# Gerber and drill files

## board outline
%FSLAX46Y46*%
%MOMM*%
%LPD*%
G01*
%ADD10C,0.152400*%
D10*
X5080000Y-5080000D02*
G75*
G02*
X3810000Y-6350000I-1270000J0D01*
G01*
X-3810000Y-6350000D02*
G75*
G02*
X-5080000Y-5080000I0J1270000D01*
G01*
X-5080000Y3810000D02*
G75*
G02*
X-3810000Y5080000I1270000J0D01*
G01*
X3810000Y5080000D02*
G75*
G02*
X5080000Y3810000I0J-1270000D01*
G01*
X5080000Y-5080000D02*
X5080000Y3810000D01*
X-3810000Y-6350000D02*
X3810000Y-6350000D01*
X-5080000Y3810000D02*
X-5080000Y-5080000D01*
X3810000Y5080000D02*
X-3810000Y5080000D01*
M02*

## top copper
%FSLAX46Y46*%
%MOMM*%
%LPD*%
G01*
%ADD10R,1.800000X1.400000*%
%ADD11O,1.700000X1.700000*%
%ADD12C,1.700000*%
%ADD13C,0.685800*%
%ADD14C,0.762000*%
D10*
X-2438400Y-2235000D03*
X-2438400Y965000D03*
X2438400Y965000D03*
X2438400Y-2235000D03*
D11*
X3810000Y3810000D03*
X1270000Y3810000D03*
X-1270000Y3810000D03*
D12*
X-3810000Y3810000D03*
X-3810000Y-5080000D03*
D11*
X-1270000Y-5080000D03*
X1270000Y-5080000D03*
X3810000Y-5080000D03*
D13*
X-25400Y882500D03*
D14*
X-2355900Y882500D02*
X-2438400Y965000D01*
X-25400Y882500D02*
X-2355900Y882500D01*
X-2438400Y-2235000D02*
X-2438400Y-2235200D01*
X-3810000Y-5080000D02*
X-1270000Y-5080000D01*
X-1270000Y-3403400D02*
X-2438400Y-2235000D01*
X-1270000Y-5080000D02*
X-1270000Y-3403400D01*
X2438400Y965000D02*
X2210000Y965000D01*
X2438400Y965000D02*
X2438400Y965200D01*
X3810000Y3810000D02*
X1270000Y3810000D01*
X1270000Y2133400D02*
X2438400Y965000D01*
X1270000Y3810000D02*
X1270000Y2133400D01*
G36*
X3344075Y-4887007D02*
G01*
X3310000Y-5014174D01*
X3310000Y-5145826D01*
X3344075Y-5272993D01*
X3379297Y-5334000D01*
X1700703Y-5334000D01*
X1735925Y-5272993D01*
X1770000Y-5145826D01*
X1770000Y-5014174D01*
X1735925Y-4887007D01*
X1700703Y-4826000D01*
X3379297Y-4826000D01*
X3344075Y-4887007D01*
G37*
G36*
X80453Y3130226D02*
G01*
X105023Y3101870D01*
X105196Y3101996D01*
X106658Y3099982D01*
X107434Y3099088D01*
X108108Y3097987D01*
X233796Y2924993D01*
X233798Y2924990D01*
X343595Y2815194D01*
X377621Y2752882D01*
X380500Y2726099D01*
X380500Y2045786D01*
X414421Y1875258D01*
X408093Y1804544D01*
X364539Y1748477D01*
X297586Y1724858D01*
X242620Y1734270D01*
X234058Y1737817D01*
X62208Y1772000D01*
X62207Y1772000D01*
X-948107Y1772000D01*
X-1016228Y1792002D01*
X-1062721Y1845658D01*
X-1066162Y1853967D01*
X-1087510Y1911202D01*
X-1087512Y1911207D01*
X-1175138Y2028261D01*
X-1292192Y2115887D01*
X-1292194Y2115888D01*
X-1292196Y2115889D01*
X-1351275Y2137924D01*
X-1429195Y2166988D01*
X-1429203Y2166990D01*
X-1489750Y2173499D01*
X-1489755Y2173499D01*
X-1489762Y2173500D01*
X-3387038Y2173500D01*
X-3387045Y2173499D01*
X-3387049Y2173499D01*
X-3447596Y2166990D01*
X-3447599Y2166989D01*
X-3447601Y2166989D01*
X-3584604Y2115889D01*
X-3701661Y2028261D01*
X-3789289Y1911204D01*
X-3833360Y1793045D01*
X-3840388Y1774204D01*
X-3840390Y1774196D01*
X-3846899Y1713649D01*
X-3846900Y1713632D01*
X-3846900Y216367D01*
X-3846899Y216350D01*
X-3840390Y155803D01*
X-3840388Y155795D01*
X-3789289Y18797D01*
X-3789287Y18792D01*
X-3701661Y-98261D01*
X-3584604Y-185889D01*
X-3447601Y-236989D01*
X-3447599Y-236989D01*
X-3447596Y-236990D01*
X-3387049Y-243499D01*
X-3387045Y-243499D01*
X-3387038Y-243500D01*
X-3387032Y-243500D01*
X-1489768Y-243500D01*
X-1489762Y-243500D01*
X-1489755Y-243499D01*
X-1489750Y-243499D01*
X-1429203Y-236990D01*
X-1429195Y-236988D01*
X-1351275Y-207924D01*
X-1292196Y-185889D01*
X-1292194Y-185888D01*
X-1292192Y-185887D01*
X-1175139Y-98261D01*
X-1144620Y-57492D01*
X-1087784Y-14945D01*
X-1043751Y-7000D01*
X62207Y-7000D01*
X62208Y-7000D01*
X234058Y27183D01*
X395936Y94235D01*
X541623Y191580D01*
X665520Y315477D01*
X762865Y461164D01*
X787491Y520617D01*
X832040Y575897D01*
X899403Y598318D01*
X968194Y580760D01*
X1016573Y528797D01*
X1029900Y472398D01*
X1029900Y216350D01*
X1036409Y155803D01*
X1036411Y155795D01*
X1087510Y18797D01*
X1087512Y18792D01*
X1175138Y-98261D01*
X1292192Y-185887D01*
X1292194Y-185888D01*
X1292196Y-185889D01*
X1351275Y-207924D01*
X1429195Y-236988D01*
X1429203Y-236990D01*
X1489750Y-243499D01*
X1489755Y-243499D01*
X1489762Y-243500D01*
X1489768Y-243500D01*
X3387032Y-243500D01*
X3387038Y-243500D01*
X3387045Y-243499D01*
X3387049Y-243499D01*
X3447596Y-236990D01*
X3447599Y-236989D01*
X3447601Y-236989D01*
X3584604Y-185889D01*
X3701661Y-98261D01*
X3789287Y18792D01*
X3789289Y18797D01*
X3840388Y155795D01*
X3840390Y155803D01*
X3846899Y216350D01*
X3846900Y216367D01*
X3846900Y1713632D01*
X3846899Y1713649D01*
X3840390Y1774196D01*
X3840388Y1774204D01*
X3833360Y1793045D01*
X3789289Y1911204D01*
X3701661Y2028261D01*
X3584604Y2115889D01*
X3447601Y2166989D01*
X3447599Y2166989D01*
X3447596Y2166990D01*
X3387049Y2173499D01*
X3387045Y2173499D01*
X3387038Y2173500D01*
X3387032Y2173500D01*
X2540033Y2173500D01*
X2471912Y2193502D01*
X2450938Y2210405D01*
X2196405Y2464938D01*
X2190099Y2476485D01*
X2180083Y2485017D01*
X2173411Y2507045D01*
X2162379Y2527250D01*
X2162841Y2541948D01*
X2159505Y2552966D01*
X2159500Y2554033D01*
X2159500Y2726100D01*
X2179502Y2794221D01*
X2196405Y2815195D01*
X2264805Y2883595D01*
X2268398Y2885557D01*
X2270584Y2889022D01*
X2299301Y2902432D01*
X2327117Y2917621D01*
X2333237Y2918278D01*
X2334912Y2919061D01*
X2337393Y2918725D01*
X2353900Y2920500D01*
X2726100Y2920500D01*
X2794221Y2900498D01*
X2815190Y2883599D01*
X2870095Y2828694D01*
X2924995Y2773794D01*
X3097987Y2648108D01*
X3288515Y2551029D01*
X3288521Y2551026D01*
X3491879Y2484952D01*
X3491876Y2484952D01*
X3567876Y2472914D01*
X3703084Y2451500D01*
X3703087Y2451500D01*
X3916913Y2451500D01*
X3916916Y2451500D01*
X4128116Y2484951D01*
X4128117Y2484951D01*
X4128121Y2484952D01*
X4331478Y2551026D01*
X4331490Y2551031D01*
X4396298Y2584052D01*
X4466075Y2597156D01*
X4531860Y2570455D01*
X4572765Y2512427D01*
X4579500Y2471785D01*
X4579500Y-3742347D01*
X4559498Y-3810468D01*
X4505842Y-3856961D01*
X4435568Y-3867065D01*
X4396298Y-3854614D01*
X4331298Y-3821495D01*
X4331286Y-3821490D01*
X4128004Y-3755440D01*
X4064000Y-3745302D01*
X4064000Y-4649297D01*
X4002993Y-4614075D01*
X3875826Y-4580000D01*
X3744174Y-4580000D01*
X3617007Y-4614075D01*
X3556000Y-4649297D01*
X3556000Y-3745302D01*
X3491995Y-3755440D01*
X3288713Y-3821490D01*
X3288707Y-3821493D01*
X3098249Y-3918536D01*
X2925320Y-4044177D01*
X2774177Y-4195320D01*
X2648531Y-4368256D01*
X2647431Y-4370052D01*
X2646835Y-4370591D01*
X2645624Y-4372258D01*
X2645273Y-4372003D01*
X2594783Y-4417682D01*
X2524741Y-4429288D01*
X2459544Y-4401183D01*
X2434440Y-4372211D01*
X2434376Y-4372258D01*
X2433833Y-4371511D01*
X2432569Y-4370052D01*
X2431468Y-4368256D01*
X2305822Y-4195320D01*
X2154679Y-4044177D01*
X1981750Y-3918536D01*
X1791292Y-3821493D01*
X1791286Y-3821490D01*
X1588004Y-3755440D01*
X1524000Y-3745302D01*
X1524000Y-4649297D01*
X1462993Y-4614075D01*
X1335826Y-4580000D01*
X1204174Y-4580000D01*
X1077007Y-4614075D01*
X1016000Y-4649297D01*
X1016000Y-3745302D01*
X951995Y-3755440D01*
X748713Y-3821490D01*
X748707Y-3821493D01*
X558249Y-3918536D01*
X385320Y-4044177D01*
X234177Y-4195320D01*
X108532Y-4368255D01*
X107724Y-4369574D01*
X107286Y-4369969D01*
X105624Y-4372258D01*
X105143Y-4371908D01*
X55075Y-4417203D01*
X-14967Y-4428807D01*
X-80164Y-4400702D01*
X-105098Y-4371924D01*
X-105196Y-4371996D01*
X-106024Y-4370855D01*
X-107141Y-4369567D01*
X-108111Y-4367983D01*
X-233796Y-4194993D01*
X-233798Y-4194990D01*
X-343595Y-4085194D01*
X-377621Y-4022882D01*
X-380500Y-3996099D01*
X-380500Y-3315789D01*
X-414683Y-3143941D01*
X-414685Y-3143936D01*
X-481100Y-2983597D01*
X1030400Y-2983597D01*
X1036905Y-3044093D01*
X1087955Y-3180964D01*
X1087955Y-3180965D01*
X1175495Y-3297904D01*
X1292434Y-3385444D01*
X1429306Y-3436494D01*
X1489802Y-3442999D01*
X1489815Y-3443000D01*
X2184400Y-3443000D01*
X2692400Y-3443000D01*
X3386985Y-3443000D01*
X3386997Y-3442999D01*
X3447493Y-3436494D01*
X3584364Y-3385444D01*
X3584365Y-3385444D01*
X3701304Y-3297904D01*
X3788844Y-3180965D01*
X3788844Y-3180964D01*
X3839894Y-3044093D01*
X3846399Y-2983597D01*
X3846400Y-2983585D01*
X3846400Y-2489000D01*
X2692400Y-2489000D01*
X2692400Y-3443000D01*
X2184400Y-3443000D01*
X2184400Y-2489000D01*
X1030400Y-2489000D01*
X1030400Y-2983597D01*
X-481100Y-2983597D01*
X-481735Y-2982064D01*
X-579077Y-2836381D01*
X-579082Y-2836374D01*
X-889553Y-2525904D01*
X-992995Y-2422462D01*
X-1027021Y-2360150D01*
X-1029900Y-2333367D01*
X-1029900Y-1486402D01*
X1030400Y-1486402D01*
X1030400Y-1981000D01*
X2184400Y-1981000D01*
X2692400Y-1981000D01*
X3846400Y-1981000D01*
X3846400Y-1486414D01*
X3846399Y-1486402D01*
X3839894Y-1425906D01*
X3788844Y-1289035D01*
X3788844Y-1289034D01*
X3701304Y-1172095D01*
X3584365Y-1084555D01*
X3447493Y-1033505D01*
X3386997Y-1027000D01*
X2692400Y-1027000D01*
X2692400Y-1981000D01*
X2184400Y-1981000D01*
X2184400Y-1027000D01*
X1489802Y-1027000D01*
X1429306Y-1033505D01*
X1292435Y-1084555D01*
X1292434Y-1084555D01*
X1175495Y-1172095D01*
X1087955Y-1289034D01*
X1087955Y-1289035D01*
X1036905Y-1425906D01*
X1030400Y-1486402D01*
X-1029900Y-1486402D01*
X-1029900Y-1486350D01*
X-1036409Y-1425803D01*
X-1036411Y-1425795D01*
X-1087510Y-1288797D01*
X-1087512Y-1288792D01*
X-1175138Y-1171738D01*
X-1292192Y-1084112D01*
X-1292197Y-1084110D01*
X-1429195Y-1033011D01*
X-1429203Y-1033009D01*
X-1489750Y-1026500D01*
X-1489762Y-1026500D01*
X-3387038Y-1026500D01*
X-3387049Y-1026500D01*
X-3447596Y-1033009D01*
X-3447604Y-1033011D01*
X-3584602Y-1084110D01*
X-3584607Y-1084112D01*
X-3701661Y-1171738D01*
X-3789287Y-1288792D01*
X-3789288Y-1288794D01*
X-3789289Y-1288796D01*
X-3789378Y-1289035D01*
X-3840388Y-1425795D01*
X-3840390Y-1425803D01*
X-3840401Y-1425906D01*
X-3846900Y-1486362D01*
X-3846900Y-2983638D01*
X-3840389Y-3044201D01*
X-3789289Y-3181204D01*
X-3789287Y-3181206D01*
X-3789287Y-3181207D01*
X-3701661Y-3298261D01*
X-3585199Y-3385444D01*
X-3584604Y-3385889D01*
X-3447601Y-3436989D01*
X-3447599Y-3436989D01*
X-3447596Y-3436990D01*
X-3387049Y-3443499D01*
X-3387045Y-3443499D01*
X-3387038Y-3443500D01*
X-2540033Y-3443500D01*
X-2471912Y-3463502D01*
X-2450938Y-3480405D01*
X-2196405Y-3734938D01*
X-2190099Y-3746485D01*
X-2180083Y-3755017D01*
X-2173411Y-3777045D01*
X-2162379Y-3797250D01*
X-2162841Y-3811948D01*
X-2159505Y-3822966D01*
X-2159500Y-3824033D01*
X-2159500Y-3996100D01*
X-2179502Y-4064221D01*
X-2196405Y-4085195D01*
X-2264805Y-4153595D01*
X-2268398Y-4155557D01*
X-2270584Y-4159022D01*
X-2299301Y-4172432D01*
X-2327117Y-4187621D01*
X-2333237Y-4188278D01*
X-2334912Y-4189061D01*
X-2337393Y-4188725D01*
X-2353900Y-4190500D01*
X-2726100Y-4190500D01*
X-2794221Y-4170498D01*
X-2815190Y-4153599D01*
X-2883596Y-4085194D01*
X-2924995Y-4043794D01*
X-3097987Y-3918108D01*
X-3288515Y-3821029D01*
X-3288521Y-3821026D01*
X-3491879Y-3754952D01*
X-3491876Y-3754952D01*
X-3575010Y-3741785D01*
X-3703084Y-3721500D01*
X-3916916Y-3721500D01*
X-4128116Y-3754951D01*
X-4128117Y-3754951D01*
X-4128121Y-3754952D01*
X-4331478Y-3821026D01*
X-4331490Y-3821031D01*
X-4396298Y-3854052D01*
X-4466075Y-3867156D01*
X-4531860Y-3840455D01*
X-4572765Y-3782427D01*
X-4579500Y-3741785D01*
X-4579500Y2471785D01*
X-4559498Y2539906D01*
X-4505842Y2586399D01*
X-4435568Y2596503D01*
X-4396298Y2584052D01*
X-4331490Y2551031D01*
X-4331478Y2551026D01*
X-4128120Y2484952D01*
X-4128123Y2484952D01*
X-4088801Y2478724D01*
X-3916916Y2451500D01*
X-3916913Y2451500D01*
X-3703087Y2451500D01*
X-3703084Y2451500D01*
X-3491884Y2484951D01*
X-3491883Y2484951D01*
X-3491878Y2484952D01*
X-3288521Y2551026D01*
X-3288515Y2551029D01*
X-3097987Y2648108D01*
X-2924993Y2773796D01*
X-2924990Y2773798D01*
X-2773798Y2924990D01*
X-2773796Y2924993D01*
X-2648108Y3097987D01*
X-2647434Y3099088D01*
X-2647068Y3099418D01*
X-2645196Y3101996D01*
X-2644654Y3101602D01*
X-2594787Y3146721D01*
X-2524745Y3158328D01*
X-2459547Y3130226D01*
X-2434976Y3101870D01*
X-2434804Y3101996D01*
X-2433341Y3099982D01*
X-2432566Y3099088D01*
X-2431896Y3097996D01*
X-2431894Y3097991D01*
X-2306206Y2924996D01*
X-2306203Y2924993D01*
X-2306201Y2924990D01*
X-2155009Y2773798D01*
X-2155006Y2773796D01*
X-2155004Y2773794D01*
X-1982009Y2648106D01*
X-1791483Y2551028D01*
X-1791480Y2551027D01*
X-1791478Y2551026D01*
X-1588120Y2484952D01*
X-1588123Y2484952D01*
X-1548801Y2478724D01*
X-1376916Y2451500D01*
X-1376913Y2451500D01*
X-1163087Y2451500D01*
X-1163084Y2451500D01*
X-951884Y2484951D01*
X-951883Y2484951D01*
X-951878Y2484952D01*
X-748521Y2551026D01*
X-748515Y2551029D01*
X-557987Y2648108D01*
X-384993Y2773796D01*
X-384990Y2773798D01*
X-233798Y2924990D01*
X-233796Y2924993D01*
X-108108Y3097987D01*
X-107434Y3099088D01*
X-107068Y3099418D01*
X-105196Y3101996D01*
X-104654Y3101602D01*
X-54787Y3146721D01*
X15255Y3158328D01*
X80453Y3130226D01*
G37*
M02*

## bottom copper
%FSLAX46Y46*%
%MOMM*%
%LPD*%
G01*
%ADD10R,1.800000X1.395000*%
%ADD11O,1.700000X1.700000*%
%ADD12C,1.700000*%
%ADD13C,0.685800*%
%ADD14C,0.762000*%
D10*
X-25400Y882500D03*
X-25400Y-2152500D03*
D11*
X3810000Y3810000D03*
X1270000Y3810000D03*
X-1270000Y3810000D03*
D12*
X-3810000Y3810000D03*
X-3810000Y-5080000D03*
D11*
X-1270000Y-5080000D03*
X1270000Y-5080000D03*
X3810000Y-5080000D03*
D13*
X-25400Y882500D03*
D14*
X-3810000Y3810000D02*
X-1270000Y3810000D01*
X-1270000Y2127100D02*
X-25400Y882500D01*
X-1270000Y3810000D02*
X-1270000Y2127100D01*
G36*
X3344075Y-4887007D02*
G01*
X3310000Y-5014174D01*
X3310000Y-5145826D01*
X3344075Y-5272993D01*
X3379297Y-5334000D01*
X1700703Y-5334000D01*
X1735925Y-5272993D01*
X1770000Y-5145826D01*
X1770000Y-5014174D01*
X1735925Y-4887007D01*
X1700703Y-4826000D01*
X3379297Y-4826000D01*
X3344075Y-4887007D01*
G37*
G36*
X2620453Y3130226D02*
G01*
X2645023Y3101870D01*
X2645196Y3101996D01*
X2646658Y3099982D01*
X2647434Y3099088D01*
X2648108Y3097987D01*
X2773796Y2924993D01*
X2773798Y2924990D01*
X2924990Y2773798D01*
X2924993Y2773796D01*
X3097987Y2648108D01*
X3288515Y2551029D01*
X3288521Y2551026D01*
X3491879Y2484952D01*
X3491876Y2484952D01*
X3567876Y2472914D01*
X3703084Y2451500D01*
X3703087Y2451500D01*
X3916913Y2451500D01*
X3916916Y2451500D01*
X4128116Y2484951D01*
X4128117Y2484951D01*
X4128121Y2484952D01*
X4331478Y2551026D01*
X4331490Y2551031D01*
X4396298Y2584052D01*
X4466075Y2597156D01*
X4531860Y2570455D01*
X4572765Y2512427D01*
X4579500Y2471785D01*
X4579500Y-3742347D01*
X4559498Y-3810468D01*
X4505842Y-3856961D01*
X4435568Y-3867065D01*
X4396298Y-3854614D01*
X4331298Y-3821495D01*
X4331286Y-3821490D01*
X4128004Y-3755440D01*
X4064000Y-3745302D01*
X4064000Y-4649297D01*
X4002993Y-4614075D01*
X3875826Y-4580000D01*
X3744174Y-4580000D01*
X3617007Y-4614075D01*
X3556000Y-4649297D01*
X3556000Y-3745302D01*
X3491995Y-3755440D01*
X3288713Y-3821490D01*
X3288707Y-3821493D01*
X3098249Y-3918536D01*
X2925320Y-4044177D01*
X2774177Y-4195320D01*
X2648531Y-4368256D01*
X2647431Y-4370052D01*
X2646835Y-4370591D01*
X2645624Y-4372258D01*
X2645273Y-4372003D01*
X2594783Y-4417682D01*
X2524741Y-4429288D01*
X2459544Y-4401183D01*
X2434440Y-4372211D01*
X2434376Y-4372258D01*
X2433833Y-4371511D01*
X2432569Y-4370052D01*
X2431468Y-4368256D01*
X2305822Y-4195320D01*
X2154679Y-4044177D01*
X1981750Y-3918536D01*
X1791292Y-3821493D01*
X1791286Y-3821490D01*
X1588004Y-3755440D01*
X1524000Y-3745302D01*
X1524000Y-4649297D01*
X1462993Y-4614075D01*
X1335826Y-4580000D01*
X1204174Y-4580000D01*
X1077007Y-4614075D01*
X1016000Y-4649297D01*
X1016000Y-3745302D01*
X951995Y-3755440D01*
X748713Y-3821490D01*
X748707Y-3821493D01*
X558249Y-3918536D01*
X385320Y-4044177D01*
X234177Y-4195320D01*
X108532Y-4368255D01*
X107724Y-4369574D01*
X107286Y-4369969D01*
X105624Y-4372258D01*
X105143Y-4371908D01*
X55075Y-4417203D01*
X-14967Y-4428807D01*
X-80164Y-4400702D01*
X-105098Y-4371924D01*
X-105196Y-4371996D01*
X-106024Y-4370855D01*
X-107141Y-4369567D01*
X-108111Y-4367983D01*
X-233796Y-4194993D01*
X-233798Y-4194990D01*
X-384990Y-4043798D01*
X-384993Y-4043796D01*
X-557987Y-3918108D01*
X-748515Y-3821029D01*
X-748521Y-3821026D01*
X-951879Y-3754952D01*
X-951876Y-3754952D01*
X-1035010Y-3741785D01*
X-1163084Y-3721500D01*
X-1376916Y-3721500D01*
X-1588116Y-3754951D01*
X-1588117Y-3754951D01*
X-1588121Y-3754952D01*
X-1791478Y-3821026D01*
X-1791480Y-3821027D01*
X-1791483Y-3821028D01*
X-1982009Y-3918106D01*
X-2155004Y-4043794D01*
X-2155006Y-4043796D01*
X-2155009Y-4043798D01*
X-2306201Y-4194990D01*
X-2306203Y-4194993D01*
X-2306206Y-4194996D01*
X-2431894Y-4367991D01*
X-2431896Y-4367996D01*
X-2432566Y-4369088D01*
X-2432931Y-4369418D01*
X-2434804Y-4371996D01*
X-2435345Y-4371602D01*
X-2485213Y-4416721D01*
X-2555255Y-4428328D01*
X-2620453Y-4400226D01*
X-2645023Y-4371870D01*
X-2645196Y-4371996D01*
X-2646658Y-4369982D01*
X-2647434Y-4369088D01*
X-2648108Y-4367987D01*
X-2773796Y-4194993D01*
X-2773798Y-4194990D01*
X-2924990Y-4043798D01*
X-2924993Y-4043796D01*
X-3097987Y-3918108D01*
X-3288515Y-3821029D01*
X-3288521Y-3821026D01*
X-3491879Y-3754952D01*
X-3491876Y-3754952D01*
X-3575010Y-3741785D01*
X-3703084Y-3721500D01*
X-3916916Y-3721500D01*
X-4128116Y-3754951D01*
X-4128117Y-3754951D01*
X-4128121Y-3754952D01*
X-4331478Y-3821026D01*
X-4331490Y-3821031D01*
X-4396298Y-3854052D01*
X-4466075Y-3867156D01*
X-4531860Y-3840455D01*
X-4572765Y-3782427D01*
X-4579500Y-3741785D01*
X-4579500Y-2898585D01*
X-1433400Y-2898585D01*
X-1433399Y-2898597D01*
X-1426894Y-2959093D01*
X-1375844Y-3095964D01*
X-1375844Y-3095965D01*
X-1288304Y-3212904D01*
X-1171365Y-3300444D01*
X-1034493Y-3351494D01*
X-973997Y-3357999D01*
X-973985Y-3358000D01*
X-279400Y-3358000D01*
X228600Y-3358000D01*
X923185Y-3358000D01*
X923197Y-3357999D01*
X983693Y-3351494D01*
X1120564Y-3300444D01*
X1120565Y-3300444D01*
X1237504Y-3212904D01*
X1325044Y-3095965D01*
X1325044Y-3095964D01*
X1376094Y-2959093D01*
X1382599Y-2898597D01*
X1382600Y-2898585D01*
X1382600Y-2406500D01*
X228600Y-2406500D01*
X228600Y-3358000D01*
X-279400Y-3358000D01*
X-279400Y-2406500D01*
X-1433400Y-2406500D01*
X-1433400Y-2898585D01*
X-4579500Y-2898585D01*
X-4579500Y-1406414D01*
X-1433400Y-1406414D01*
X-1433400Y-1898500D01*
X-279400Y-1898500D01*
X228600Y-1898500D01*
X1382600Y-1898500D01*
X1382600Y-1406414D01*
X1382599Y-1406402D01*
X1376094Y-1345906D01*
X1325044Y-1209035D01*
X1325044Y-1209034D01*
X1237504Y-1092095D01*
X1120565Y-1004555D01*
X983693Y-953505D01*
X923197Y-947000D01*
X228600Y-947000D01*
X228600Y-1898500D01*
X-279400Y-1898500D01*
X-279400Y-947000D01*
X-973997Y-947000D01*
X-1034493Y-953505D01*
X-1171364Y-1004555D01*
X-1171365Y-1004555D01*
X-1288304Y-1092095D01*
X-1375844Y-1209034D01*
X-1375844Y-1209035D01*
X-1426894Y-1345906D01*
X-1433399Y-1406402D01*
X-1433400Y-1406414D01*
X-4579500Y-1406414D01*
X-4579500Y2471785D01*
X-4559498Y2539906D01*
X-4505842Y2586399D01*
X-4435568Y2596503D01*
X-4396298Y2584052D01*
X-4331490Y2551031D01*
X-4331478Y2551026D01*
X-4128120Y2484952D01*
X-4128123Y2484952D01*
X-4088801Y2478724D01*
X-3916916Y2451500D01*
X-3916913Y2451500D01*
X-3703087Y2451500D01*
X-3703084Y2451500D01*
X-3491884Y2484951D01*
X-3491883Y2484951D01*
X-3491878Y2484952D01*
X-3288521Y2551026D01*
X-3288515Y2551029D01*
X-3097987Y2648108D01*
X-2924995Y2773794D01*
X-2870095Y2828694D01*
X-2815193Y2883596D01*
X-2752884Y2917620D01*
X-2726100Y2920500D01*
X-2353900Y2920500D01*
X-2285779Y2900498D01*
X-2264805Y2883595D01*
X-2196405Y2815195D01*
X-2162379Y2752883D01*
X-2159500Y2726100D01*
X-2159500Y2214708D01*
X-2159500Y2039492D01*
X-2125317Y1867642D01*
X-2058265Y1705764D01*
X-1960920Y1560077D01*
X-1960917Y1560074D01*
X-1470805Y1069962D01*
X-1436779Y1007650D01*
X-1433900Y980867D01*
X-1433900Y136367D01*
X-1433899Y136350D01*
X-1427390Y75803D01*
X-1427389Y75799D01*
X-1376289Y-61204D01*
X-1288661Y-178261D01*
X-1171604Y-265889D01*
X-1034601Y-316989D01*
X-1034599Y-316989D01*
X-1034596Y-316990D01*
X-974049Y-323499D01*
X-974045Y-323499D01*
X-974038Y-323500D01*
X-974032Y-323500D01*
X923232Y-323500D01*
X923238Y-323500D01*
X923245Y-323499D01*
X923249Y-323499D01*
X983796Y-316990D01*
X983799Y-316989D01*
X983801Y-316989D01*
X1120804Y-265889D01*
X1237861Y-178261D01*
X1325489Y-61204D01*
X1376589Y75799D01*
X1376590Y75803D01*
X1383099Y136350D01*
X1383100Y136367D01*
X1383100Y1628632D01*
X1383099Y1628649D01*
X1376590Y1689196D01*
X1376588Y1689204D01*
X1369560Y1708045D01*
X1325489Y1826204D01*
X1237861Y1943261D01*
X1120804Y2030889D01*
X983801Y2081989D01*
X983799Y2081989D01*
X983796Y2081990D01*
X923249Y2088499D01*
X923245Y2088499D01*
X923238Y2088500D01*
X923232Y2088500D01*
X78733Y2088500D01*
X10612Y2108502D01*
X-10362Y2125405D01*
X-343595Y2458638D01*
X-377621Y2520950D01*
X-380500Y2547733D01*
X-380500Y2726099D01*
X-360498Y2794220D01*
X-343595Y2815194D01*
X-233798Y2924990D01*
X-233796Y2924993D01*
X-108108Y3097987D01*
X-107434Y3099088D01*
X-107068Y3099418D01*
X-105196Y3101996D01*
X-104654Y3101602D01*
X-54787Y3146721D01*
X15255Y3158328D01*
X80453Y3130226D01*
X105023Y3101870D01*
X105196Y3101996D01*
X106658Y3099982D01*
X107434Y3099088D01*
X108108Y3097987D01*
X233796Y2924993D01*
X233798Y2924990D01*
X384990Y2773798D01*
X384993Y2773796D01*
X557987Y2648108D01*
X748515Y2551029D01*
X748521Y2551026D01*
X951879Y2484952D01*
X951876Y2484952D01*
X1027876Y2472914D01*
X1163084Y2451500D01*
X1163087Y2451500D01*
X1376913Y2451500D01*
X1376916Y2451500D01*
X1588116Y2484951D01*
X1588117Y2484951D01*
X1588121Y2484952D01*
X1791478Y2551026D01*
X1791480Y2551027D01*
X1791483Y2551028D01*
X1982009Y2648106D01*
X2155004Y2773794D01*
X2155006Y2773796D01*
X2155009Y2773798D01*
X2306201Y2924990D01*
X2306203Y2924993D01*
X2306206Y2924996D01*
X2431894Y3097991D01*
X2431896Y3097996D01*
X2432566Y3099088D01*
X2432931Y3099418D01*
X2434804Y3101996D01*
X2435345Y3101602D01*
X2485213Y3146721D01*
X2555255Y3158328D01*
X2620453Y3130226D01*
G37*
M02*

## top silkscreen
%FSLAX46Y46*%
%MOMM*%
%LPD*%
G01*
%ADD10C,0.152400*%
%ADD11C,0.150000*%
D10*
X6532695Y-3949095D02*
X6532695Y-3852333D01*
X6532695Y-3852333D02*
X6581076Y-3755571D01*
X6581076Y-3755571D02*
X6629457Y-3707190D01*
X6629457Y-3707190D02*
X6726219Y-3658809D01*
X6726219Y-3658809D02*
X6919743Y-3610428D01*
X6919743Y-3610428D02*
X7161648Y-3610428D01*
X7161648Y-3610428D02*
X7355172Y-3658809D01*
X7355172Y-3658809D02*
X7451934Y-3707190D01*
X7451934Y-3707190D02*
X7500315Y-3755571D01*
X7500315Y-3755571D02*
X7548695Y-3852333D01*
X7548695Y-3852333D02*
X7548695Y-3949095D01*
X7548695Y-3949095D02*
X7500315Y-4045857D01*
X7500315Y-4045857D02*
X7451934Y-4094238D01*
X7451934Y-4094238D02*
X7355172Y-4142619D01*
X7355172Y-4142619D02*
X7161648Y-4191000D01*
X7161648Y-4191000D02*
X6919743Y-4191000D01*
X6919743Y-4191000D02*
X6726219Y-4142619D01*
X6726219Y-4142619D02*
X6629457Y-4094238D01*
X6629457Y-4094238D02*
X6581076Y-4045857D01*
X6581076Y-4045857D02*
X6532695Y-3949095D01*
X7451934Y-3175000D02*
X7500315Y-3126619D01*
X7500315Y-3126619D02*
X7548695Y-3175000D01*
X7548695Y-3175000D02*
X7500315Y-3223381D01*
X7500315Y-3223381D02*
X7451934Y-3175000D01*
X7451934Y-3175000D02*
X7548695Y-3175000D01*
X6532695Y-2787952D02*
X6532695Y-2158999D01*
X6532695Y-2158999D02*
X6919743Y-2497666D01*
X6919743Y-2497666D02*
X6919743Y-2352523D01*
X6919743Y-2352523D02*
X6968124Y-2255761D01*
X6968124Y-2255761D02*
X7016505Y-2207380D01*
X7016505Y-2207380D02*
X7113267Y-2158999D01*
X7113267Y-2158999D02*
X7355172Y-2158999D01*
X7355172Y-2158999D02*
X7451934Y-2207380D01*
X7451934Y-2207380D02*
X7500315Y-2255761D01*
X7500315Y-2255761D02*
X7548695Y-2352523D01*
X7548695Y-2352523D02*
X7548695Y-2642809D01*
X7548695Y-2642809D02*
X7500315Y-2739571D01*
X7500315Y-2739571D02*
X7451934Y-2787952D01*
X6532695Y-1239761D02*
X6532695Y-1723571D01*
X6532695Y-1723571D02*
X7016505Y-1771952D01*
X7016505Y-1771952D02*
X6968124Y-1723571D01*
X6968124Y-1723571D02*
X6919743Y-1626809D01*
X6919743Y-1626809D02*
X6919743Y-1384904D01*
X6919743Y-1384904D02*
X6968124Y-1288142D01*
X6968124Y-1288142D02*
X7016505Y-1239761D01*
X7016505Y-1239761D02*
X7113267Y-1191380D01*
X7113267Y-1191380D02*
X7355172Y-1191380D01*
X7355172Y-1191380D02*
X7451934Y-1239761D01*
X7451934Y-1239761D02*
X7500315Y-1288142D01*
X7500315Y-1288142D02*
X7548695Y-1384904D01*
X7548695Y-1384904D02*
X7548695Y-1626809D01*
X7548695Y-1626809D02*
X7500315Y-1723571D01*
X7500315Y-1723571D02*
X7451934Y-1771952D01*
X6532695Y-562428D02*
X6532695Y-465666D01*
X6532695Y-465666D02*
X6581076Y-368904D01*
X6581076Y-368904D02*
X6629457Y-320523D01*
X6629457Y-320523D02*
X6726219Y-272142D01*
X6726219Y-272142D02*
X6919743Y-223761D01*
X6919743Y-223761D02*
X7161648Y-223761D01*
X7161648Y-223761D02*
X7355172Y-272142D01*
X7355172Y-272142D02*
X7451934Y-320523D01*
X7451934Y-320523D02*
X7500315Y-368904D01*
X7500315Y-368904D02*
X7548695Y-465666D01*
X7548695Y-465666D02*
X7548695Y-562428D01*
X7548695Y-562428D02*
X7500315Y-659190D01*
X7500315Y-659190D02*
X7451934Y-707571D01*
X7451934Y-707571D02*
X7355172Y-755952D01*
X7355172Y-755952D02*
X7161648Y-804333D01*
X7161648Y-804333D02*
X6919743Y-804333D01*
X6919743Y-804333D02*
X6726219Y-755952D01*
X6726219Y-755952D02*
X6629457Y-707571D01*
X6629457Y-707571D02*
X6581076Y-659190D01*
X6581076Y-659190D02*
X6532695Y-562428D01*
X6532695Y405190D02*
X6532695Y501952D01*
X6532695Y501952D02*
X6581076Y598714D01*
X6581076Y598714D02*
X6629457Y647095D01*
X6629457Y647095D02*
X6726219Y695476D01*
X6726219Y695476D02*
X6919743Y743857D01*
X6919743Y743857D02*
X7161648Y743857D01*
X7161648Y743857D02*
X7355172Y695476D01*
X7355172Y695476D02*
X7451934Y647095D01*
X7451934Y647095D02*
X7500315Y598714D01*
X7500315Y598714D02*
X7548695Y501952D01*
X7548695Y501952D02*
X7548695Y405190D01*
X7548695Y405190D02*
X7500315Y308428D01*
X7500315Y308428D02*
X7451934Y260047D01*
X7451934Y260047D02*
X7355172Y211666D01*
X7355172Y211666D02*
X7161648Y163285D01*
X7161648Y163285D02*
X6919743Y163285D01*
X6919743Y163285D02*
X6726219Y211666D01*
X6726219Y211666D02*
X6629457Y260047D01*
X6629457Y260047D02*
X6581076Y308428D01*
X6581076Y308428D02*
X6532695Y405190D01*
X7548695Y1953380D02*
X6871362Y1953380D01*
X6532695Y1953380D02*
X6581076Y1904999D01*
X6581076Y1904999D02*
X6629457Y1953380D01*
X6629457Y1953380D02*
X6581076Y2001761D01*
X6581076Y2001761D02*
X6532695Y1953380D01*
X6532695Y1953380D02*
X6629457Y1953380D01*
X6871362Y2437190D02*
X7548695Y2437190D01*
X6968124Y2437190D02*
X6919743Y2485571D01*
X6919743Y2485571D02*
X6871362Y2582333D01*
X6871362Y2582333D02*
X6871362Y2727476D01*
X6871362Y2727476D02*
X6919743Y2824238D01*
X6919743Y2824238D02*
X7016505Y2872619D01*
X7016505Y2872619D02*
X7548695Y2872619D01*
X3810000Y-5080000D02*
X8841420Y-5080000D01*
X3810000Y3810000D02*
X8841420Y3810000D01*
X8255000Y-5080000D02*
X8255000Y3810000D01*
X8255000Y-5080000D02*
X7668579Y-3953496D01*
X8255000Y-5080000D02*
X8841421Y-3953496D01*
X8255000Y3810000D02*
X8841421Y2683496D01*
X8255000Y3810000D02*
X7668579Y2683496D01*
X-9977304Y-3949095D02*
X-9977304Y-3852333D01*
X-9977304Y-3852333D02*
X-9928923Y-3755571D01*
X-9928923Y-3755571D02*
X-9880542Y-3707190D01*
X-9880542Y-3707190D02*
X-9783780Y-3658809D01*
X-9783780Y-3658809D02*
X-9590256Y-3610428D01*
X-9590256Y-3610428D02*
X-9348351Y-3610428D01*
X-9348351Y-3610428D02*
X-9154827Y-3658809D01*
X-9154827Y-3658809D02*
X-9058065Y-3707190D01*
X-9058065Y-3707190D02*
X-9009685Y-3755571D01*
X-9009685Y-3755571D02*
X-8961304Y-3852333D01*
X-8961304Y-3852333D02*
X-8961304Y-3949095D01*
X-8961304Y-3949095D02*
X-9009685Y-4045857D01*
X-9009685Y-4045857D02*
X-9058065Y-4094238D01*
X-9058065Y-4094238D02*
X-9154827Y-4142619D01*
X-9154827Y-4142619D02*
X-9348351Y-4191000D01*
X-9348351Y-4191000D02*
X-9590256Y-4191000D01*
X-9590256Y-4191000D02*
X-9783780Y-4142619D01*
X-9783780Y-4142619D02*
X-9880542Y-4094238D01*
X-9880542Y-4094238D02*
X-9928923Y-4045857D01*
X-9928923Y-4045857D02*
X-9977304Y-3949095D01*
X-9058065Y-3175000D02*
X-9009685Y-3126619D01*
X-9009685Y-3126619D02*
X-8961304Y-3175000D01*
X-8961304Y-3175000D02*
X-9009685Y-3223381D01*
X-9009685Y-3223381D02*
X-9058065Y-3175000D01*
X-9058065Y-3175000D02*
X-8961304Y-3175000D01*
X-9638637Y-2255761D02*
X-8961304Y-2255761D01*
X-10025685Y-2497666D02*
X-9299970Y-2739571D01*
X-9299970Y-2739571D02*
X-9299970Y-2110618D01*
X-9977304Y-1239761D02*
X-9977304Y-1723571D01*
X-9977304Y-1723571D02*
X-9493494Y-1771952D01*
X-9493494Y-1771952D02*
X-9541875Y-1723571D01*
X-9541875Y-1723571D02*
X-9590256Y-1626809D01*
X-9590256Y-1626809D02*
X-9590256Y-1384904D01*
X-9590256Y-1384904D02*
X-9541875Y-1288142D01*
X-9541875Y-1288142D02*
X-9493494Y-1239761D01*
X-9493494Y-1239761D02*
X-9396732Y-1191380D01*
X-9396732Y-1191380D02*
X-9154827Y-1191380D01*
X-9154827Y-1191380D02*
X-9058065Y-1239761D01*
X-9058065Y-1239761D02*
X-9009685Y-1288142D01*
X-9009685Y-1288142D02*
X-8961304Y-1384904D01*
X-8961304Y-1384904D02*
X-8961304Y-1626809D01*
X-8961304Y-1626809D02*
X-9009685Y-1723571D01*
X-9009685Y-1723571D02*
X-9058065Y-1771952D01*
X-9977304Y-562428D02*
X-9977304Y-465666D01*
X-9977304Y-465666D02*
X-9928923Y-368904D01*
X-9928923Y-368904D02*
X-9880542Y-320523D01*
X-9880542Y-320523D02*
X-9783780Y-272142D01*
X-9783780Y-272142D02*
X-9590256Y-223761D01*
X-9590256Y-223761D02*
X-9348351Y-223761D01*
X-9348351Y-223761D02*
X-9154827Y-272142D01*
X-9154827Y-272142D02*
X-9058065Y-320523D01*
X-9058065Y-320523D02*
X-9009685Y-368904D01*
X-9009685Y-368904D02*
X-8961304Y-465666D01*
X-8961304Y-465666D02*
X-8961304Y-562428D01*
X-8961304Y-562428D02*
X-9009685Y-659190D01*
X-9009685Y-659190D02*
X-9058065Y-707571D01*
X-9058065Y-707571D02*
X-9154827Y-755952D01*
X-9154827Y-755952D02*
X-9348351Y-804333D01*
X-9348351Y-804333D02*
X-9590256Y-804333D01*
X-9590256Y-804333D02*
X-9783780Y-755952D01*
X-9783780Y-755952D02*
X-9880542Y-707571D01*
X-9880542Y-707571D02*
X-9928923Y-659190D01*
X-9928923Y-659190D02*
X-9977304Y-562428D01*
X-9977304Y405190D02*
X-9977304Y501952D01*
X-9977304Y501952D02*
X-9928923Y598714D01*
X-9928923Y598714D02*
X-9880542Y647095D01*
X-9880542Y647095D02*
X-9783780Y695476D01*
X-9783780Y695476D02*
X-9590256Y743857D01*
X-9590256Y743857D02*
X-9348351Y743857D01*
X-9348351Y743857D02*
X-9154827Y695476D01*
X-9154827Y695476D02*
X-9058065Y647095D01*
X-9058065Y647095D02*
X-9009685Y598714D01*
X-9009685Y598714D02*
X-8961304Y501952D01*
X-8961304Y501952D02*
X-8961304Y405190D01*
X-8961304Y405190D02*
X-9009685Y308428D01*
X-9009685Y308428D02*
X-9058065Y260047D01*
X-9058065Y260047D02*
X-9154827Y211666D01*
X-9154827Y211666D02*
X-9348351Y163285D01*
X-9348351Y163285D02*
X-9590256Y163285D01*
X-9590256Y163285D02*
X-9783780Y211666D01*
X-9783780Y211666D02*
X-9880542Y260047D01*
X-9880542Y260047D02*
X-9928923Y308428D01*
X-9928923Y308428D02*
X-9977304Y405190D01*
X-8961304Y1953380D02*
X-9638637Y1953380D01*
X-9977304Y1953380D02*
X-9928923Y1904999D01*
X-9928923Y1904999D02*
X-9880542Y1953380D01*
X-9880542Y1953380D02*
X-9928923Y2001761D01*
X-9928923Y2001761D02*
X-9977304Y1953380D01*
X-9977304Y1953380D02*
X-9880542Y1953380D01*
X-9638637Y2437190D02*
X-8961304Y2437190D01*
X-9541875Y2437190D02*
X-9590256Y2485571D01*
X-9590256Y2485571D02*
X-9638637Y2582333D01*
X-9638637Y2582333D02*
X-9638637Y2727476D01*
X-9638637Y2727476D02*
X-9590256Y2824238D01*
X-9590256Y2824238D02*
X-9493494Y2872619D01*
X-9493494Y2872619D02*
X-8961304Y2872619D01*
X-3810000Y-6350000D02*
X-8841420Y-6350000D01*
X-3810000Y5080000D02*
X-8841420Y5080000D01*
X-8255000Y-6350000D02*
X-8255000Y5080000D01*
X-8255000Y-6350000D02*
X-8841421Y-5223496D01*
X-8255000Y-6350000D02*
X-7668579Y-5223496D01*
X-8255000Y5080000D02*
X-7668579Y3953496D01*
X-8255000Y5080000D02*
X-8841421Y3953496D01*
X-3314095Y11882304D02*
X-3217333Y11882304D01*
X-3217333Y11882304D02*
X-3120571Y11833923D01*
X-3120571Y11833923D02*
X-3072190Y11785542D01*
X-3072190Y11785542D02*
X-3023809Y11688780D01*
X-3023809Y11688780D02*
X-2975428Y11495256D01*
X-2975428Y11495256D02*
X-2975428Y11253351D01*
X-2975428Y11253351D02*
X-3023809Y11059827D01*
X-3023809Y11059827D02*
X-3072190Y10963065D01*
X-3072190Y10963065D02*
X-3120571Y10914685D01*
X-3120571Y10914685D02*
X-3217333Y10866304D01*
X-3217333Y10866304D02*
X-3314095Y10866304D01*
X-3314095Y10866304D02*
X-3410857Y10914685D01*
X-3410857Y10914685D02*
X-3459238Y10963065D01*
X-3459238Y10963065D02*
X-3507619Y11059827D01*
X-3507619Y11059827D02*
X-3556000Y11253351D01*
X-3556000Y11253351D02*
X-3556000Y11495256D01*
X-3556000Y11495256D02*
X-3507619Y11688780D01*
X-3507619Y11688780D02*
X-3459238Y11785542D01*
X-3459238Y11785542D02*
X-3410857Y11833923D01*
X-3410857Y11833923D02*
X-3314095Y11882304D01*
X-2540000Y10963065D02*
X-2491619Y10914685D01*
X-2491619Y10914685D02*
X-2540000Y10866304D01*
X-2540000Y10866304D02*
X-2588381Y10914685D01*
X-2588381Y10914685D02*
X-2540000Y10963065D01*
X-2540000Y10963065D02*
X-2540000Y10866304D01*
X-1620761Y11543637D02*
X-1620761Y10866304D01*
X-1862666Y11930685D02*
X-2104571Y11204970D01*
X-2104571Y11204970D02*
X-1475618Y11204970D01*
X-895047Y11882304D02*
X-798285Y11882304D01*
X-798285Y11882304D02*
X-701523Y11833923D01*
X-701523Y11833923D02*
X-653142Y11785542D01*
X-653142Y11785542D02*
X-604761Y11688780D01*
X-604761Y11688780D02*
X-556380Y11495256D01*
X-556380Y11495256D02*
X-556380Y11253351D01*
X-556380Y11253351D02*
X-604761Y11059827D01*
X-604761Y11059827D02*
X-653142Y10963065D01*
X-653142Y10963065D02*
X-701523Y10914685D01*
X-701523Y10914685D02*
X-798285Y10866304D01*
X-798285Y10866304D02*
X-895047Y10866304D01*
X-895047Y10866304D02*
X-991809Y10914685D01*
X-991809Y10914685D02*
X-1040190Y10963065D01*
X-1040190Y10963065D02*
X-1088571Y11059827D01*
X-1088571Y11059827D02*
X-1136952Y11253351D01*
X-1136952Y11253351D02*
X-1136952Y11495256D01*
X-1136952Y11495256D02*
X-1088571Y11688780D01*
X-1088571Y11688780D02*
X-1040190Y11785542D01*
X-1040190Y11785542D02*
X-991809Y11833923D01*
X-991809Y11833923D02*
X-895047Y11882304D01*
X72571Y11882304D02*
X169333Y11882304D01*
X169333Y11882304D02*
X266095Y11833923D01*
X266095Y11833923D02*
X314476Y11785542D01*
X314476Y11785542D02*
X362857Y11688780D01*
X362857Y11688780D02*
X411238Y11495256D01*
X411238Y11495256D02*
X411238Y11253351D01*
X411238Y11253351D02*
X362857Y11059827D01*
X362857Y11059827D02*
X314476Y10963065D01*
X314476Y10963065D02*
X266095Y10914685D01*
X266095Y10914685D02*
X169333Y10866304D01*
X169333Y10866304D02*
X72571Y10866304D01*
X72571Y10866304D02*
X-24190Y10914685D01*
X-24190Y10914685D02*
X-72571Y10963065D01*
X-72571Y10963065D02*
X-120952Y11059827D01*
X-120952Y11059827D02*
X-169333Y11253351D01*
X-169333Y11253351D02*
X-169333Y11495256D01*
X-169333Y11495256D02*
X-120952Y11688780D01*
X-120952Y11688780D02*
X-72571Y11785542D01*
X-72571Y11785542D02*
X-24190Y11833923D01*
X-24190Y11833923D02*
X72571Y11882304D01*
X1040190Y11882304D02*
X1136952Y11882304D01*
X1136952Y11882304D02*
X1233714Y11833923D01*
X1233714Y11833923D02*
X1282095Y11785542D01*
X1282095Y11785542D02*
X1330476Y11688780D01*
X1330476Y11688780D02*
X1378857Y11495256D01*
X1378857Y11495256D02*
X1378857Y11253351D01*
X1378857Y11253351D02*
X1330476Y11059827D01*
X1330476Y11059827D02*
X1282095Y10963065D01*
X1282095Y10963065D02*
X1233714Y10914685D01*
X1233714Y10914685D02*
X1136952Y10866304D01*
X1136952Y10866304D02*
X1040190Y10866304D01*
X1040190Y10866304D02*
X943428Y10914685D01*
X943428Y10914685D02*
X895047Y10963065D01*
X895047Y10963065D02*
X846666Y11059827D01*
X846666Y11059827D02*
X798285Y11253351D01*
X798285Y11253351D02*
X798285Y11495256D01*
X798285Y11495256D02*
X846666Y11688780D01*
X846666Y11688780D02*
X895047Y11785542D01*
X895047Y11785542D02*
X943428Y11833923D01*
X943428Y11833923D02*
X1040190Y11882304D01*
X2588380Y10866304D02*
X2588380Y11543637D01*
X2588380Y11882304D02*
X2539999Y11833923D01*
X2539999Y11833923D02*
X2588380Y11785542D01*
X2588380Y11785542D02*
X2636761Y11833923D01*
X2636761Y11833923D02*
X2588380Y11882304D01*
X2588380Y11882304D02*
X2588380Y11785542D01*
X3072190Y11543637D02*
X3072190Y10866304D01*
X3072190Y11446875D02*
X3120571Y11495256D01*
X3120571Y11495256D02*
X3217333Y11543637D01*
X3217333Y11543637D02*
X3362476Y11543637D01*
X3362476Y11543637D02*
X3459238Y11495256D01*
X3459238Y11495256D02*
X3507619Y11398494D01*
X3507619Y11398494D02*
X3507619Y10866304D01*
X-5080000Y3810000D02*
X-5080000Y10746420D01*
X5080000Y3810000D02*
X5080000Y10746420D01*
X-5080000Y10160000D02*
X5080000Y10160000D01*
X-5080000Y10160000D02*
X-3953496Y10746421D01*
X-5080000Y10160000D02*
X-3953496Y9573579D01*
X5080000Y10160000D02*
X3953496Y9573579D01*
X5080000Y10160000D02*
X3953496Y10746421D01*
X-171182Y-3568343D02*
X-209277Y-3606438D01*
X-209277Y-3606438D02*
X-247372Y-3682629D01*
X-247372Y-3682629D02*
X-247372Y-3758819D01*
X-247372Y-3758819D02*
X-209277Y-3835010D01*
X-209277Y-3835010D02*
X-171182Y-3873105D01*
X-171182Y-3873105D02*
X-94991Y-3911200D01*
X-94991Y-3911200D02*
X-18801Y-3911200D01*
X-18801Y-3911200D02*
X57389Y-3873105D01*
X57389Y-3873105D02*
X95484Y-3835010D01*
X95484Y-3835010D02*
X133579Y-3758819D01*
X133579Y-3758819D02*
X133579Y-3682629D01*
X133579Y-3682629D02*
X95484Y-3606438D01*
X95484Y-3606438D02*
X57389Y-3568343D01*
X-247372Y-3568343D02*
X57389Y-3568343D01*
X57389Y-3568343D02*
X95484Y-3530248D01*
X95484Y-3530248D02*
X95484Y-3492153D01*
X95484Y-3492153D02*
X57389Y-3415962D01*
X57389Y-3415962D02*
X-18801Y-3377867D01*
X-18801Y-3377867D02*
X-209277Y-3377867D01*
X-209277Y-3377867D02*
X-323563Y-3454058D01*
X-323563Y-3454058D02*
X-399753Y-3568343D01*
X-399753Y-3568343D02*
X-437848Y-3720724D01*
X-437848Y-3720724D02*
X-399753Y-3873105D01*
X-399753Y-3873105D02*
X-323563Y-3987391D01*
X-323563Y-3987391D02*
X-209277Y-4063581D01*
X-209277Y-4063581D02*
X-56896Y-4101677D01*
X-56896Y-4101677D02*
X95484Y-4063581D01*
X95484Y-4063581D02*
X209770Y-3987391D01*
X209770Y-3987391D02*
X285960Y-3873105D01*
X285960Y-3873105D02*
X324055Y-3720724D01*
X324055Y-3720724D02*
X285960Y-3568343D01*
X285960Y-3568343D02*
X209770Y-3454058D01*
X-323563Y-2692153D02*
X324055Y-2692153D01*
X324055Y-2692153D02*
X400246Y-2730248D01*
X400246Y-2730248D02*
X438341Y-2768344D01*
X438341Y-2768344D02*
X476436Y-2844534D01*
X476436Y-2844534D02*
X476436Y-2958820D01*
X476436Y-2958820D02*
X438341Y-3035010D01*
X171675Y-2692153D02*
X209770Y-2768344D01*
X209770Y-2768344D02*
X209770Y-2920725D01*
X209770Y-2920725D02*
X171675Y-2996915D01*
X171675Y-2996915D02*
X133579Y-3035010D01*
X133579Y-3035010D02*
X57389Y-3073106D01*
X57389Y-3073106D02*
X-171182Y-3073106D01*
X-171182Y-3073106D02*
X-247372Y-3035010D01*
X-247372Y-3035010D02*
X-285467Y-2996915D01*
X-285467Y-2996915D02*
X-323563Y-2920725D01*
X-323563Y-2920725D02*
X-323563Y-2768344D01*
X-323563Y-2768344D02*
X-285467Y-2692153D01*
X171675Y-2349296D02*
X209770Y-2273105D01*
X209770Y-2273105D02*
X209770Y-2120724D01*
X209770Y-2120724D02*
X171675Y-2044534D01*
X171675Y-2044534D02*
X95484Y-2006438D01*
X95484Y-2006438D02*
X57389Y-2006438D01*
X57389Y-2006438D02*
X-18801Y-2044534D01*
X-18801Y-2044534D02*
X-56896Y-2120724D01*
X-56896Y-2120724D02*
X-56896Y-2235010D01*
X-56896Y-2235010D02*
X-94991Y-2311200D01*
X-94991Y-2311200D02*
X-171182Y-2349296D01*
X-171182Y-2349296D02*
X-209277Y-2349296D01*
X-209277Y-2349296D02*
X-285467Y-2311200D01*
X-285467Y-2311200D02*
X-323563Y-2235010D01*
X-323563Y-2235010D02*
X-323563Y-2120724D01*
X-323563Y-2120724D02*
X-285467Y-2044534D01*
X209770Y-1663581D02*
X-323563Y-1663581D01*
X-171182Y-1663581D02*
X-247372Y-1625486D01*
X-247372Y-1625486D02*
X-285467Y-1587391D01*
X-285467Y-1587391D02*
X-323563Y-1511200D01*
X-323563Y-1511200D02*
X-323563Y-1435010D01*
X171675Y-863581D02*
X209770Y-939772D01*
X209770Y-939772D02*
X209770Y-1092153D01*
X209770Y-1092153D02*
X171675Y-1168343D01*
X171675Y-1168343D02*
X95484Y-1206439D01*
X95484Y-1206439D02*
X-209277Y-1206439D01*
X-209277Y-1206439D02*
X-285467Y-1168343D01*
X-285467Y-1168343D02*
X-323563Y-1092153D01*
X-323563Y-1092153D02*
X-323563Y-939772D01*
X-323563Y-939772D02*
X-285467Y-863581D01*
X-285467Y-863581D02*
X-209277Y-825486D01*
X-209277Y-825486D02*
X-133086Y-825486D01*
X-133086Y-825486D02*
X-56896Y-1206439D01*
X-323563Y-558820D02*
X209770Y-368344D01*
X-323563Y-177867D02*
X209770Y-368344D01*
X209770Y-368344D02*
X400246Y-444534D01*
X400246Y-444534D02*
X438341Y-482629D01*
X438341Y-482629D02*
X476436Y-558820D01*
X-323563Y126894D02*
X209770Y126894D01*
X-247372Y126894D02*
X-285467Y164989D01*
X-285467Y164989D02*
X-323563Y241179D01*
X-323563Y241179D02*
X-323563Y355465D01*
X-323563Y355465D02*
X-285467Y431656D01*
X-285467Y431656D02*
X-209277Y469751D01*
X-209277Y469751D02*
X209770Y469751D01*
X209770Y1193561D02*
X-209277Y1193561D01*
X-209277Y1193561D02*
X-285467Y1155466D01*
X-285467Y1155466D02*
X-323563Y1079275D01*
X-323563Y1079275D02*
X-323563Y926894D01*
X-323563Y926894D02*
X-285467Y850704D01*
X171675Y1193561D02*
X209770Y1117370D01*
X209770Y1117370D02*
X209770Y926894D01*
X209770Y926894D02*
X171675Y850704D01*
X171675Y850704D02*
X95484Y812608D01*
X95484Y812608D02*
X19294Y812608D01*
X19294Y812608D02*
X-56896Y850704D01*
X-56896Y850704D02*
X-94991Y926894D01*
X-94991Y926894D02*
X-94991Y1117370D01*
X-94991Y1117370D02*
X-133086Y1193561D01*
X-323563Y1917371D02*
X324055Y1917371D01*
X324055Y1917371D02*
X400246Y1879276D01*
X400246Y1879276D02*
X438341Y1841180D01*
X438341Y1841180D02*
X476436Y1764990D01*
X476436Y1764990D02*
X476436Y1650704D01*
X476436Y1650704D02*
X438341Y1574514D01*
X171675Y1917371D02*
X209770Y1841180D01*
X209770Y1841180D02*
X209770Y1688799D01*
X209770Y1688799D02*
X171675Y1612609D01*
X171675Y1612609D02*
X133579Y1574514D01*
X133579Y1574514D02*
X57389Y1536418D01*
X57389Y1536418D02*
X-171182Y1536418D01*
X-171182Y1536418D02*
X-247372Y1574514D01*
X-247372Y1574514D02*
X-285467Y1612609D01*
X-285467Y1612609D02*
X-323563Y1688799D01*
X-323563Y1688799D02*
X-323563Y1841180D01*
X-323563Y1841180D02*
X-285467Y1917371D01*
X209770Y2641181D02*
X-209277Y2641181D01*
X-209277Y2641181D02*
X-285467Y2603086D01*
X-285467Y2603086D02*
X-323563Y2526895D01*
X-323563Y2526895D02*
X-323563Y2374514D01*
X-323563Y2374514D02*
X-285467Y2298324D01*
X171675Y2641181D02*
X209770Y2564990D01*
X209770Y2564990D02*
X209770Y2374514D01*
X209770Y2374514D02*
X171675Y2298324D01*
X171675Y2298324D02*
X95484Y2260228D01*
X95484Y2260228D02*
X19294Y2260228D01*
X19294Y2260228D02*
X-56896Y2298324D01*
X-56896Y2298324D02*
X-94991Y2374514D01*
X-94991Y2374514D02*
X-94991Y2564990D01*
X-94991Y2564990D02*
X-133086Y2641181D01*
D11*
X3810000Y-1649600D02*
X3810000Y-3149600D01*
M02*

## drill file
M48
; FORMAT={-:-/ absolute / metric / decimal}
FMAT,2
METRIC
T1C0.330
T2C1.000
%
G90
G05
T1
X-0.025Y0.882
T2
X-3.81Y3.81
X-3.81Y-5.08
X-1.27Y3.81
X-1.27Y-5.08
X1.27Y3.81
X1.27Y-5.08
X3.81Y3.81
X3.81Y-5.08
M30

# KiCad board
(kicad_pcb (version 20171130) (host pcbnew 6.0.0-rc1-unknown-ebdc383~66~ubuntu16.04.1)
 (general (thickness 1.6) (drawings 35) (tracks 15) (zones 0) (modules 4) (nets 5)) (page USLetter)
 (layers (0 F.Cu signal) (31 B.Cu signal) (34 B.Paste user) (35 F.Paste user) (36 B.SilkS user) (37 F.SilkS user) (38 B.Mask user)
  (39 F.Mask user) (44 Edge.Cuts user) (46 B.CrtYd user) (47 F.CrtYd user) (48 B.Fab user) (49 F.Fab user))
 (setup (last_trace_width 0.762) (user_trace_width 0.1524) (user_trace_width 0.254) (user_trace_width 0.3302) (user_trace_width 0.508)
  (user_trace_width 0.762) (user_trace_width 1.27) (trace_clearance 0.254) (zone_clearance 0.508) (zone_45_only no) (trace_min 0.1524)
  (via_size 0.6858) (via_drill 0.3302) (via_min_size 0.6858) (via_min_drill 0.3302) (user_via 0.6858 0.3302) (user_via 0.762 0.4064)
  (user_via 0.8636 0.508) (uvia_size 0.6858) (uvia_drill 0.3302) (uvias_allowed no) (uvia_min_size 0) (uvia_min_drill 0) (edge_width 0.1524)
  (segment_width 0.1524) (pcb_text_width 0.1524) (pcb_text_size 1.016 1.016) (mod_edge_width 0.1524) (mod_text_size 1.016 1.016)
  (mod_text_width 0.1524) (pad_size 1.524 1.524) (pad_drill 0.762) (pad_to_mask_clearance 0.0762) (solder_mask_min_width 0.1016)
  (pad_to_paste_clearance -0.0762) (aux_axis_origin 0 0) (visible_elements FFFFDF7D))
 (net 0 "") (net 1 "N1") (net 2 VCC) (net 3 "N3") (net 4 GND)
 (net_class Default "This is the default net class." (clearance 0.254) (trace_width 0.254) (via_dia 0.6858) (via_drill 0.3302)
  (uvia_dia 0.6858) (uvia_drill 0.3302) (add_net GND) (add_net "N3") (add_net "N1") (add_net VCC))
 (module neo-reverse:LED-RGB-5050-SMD (layer F.Cu) (at 0 0.635)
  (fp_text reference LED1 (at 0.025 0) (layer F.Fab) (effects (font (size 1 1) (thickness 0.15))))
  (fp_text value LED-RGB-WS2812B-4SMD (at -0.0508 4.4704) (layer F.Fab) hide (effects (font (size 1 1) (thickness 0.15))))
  (fp_line (start 3.81 1.0146) (end 3.81 2.5146) (layer F.SilkS) (width 0.15))
  (pad 4 smd rect (at -2.4384 1.6) (size 1.8 1.4) (layers F.Cu F.Paste F.Mask) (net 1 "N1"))
  (pad 3 smd rect (at -2.4384 -1.6) (size 1.8 1.4) (layers F.Cu F.Paste F.Mask) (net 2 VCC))
  (pad 2 smd rect (at 2.4384 -1.6) (size 1.8 1.4) (layers F.Cu F.Paste F.Mask) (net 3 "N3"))
  (pad 1 smd rect (at 2.4384 1.6) (size 1.8 1.4) (layers F.Cu F.Paste F.Mask) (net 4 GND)))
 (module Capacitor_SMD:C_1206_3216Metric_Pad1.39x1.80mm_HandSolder (layer B.Cu) (at -0.0254 0.635 270)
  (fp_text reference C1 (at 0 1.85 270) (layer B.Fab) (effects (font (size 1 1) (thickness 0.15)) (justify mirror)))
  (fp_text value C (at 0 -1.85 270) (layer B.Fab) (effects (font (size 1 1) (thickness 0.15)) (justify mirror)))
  (pad 1 smd rect (at -1.5175 0 270) (size 1.395 1.8) (layers B.Cu B.Paste B.Mask) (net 2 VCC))
  (pad 2 smd rect (at 1.5175 0 270) (size 1.395 1.8) (layers B.Cu B.Paste B.Mask) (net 4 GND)))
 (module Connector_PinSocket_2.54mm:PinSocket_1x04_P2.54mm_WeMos (layer F.Cu) (at -3.81 -3.81 90)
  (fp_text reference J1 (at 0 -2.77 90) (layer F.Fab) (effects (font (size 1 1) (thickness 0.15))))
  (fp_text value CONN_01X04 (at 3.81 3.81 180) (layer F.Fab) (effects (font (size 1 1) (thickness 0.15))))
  (pad 4 thru_hole oval (at 0 7.62 90) (size 1.7 1.7) (drill 1) (layers *.Cu *.Mask) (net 3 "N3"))
  (pad 3 thru_hole oval (at 0 5.08 90) (size 1.7 1.7) (drill 1) (layers *.Cu *.Mask) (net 3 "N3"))
  (pad 2 thru_hole oval (at 0 2.54 90) (size 1.7 1.7) (drill 1) (layers *.Cu *.Mask) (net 2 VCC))
  (pad 1 thru_hole circle (at 0 0 90) (size 1.7 1.7) (drill 1) (layers *.Cu *.Mask) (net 2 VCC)))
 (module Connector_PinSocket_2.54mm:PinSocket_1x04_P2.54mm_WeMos (layer F.Cu) (at -3.81 5.08 90)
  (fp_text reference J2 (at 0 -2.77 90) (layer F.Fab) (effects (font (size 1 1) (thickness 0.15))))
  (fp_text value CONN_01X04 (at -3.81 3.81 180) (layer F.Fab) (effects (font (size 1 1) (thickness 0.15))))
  (pad 1 thru_hole circle (at 0 0 90) (size 1.7 1.7) (drill 1) (layers *.Cu *.Mask) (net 1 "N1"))
  (pad 2 thru_hole oval (at 0 2.54 90) (size 1.7 1.7) (drill 1) (layers *.Cu *.Mask) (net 1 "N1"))
  (pad 3 thru_hole oval (at 0 5.08 90) (size 1.7 1.7) (drill 1) (layers *.Cu *.Mask) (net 4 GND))
  (pad 4 thru_hole oval (at 0 7.62 90) (size 1.7 1.7) (drill 1) (layers *.Cu *.Mask) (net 4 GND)))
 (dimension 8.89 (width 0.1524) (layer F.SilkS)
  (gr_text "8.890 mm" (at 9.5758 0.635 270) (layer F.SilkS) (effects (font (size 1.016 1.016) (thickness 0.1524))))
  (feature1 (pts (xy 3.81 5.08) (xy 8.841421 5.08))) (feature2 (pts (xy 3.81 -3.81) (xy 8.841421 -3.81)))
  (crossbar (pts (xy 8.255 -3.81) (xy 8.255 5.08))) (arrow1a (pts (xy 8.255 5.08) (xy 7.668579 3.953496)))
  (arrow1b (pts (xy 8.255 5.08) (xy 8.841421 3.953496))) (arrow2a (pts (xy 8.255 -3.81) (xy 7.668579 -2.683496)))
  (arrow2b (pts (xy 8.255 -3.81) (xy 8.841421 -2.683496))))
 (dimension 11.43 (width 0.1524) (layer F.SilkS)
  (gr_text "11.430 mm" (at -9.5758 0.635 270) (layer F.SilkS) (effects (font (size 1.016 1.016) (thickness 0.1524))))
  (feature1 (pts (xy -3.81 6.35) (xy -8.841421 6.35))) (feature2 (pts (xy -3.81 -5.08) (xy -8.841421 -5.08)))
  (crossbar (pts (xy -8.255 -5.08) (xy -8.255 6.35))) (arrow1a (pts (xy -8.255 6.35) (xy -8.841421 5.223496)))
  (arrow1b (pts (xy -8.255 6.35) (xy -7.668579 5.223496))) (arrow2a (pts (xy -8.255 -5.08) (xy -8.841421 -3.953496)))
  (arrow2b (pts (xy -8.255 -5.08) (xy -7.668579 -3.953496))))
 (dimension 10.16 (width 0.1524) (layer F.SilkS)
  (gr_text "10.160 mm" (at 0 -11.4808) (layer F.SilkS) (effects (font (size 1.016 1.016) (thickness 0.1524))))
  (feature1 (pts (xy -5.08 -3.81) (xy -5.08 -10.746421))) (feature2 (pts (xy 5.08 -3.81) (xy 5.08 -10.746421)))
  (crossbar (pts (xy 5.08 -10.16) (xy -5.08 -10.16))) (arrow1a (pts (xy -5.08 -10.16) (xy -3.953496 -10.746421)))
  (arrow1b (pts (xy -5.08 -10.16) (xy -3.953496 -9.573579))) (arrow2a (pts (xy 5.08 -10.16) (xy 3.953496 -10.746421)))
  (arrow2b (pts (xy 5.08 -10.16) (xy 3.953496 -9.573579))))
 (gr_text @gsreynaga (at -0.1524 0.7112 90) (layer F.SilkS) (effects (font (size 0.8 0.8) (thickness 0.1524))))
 (gr_arc (start 3.81 5.08) (end 3.81 6.35) (angle -90) (layer Edge.Cuts) (width 0.1524))
 (gr_arc (start -3.81 5.08) (end -5.08 5.08) (angle -90) (layer Edge.Cuts) (width 0.1524))
 (gr_arc (start -3.81 -3.81) (end -3.81 -5.08) (angle -90) (layer Edge.Cuts) (width 0.1524))
 (gr_arc (start 3.81 -3.81) (end 5.08 -3.81) (angle -90) (layer Edge.Cuts) (width 0.1524))
 (gr_line (start 5.08 5.08) (end 5.08 -3.81) (layer Edge.Cuts) (width 0.1524))
 (gr_line (start -3.81 6.35) (end 3.81 6.35) (layer Edge.Cuts) (width 0.1524))
 (gr_line (start -5.08 -3.81) (end -5.08 5.08) (layer Edge.Cuts) (width 0.1524))
 (gr_line (start 3.81 -5.08) (end -3.81 -5.08) (layer Edge.Cuts) (width 0.1524))
 (via (at -0.0254 -0.8825) (size 0.6858) (drill 0.3302) (layers F.Cu B.Cu) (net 2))
 (segment (start -3.81 -3.81) (end -1.27 -3.81) (width 0.762) (layer B.Cu) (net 2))
 (segment (start -1.27 -2.1271) (end -0.0254 -0.8825) (width 0.762) (layer B.Cu) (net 2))
 (segment (start -1.27 -3.81) (end -1.27 -2.1271) (width 0.762) (layer B.Cu) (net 2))
 (segment (start -2.3559 -0.8825) (end -2.4384 -0.965) (width 0.762) (layer F.Cu) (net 2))
 (segment (start -0.0254 -0.8825) (end -2.3559 -0.8825) (width 0.762) (layer F.Cu) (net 2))
 (segment (start -2.4384 2.235) (end -2.4384 2.2352) (width 0.762) (layer F.Cu) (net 1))
 (segment (start -3.81 5.08) (end -1.27 5.08) (width 0.762) (layer F.Cu) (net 1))
 (segment (start -1.27 3.4034) (end -2.4384 2.235) (width 0.762) (layer F.Cu) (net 1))
 (segment (start -1.27 5.08) (end -1.27 3.4034) (width 0.762) (layer F.Cu) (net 1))
 (segment (start 2.4384 -0.965) (end 2.21 -0.965) (width 0.762) (layer F.Cu) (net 3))
 (segment (start 2.4384 -0.965) (end 2.4384 -0.9652) (width 0.762) (layer F.Cu) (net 3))
 (segment (start 3.81 -3.81) (end 1.27 -3.81) (width 0.762) (layer F.Cu) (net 3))
 (segment (start 1.27 -2.1334) (end 2.4384 -0.965) (width 0.762) (layer F.Cu) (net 3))
 (segment (start 1.27 -3.81) (end 1.27 -2.1334) (width 0.762) (layer F.Cu) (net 3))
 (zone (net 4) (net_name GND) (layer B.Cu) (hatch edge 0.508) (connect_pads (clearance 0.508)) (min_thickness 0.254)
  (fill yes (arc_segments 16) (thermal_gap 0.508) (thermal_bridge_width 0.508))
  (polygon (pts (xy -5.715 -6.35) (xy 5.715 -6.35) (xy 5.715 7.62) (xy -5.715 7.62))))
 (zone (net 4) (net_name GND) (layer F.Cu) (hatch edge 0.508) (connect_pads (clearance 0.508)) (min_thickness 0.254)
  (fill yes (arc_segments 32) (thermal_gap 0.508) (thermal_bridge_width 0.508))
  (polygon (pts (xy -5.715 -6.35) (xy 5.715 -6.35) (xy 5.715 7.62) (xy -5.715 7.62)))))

